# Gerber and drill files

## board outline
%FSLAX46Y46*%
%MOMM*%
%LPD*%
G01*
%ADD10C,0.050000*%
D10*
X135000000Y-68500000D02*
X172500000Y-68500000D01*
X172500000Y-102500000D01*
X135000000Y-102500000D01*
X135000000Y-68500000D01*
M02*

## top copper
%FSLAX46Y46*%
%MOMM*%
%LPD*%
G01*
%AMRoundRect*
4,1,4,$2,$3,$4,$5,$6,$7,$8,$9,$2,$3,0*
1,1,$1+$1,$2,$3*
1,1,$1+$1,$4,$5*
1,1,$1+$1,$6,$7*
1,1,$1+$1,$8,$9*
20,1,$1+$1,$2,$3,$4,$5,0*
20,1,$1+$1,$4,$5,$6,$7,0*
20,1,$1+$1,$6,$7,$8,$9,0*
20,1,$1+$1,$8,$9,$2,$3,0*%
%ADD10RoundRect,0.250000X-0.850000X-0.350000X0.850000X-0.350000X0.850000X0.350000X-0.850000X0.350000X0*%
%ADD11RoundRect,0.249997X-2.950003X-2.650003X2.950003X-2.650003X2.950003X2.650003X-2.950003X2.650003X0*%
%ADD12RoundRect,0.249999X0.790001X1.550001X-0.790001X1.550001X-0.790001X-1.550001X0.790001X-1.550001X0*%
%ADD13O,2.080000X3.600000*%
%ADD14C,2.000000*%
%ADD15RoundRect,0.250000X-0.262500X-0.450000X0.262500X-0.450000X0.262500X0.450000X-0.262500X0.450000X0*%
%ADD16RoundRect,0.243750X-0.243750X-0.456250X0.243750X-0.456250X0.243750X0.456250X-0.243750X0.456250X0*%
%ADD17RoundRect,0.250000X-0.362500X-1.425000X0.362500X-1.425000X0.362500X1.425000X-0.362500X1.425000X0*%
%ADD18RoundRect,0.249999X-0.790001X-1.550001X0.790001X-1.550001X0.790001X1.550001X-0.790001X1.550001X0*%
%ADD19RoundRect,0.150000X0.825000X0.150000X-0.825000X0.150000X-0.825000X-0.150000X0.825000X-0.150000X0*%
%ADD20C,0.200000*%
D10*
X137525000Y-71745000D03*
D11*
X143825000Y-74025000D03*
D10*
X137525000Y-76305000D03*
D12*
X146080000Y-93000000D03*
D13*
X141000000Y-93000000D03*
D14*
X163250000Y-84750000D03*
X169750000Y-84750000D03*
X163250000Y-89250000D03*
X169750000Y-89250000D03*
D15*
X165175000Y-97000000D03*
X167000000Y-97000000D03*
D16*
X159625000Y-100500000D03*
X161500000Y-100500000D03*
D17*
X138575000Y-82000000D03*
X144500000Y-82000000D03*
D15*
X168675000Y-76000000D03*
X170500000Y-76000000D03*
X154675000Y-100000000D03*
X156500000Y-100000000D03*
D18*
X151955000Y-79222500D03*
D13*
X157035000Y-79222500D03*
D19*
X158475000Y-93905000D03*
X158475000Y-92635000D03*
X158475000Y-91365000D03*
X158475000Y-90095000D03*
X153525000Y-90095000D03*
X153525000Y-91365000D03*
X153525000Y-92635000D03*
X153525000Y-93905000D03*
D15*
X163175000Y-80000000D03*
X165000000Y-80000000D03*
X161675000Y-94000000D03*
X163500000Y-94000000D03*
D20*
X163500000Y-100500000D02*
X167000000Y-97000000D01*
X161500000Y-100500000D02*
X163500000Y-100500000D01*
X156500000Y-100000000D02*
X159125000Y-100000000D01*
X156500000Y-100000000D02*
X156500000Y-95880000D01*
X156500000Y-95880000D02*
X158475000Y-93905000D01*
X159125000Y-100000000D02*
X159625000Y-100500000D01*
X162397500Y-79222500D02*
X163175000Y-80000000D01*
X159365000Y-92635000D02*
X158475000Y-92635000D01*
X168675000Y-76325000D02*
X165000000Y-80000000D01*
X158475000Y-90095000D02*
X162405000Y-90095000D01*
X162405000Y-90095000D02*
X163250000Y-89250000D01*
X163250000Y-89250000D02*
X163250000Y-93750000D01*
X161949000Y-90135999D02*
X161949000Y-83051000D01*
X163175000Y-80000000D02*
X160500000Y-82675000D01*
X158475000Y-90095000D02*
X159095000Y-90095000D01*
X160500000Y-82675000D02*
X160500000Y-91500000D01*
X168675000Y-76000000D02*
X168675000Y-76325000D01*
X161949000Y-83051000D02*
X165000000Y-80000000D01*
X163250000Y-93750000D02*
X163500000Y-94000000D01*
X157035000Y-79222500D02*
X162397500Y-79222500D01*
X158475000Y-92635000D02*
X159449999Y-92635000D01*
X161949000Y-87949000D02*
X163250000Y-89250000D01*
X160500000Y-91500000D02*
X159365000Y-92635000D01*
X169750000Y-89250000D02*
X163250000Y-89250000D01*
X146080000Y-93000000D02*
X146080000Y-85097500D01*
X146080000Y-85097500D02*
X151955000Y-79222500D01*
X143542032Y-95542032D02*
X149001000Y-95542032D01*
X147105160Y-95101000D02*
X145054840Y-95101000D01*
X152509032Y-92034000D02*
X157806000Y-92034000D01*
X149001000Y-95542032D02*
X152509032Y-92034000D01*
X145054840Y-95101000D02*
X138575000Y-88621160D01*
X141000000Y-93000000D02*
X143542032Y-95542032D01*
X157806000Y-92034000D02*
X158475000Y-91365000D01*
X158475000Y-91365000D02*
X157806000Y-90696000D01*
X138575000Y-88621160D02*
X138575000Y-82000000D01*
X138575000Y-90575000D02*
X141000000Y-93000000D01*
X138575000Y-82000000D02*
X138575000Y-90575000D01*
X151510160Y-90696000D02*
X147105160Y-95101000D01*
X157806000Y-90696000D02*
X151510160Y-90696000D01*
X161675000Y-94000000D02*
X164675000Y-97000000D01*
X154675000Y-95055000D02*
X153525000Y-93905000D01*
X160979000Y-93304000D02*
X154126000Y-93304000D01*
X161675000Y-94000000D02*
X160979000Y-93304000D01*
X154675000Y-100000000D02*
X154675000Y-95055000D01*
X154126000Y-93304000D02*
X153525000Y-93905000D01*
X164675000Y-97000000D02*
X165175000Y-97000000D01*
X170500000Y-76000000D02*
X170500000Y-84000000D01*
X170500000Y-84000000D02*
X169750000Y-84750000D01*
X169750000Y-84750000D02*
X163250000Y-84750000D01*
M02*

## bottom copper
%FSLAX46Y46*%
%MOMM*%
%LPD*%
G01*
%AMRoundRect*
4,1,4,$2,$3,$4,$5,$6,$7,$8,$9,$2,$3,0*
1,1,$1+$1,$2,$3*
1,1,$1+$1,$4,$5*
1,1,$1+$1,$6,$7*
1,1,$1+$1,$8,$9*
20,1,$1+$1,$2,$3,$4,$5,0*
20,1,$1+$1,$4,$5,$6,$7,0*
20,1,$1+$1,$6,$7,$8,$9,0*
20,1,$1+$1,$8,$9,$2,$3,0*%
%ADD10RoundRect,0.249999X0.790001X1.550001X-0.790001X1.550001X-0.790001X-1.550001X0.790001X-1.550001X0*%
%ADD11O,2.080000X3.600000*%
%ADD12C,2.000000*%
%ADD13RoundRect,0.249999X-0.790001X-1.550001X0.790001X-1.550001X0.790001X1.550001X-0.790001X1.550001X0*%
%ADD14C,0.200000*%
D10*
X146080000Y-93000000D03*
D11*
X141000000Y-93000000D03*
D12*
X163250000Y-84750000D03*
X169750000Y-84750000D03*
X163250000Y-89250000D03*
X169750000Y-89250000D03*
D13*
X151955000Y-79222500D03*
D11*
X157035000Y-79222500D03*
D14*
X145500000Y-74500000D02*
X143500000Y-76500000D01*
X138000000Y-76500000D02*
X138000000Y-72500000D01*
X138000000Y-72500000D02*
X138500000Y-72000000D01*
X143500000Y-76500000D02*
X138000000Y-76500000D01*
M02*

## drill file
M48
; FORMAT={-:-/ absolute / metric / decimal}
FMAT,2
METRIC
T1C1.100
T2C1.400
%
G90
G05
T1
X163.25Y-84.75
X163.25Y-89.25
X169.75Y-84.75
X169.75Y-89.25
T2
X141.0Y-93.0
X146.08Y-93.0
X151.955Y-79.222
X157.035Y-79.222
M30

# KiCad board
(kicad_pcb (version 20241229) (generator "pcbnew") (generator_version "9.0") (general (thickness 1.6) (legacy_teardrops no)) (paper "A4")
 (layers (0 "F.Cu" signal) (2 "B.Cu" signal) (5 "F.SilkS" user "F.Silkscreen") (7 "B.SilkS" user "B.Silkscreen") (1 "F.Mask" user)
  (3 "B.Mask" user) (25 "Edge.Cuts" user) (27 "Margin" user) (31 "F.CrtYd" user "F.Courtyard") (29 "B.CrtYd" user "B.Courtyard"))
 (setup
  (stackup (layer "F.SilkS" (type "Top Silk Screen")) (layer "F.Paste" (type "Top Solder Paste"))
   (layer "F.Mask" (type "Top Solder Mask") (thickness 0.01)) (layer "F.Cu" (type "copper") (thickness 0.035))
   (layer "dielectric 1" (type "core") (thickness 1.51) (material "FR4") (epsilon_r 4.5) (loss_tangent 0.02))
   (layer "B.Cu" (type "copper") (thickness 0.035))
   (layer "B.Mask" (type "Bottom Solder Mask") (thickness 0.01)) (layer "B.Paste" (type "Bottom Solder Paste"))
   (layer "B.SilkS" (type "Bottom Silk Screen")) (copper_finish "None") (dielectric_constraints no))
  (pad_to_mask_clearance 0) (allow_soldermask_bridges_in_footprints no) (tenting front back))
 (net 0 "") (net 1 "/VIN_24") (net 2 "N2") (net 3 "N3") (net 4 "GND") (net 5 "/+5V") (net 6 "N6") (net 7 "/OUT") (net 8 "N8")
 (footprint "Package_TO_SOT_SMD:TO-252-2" (layer "F.Cu") (at 142.565 74.025)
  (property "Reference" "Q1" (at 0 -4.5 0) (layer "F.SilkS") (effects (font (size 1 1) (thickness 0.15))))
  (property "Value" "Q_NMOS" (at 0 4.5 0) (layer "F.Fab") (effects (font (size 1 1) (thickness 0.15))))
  (pad "" smd roundrect (at -0.415 -1.525) (size 3.05 2.75) (layers "F.Paste") (roundrect_rratio 0.090909))
  (pad "" smd roundrect (at -0.415 1.525) (size 3.05 2.75) (layers "F.Paste") (roundrect_rratio 0.090909))
  (pad "" smd roundrect (at 2.935 -1.525) (size 3.05 2.75) (layers "F.Paste") (roundrect_rratio 0.090909))
  (pad "" smd roundrect (at 2.935 1.525) (size 3.05 2.75) (layers "F.Paste") (roundrect_rratio 0.090909))
  (pad "1" smd roundrect (at -5.04 -2.28) (size 2.2 1.2) (layers "F.Cu" "F.Mask" "F.Paste") (roundrect_rratio 0.208333))
  (pad "2" smd roundrect (at 1.26 0) (size 6.4 5.8) (layers "F.Cu" "F.Mask") (roundrect_rratio 0.043103))
  (pad "3" smd roundrect (at -5.04 2.28) (size 2.2 1.2) (layers "F.Cu" "F.Mask" "F.Paste") (roundrect_rratio 0.208333)))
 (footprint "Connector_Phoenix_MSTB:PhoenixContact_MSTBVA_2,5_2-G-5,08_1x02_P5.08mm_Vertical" (layer "F.Cu") (at 146.08 93 180)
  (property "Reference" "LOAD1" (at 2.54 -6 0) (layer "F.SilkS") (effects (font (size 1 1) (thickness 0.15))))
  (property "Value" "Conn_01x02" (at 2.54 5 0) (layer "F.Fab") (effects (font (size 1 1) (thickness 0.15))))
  (pad "1" thru_hole roundrect (at 0 0 180) (size 2.08 3.6) (drill 1.4) (layers "*.Cu" "*.Mask") (remove_unused_layers no)
   (roundrect_rratio 0.120192) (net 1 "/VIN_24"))
  (pad "2" thru_hole oval (at 5.08 0 180) (size 2.08 3.6) (drill 1.4) (layers "*.Cu" "*.Mask") (remove_unused_layers no) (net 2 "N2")))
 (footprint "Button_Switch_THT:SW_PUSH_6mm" (layer "F.Cu") (at 163.25 84.75)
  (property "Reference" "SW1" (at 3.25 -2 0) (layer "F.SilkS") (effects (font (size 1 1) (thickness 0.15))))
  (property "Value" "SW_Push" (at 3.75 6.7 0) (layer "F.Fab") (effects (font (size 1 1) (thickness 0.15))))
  (pad "1" thru_hole circle (at 0 0 90) (size 2 2) (drill 1.1) (layers "*.Cu" "*.Mask") (remove_unused_layers no) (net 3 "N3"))
  (pad "1" thru_hole circle (at 6.5 0 90) (size 2 2) (drill 1.1) (layers "*.Cu" "*.Mask") (remove_unused_layers no) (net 3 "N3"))
  (pad "2" thru_hole circle (at 0 4.5 90) (size 2 2) (drill 1.1) (layers "*.Cu" "*.Mask") (remove_unused_layers no) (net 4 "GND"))
  (pad "2" thru_hole circle (at 6.5 4.5 90) (size 2 2) (drill 1.1) (layers "*.Cu" "*.Mask") (remove_unused_layers no) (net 4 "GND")))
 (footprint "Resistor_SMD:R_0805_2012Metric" (layer "F.Cu") (at 166.0875 97)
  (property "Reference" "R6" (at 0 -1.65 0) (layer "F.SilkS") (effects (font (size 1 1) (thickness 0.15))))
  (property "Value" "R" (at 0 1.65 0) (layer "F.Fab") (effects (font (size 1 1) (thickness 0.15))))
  (pad "1" smd roundrect (at -0.9125 0) (size 1.025 1.4) (layers "F.Cu" "F.Mask" "F.Paste") (roundrect_rratio 0.243902) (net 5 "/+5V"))
  (pad "2" smd roundrect (at 0.9125 0) (size 1.025 1.4) (layers "F.Cu" "F.Mask" "F.Paste") (roundrect_rratio 0.243902) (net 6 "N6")))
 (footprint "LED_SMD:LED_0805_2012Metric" (layer "F.Cu") (at 160.5625 100.5)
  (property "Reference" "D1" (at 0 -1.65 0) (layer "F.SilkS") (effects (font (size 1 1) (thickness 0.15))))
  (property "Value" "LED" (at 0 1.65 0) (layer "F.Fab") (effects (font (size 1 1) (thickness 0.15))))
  (pad "1" smd roundrect (at -0.9375 0) (size 0.975 1.4) (layers "F.Cu" "F.Mask" "F.Paste") (roundrect_rratio 0.25) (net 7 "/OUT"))
  (pad "2" smd roundrect (at 0.9375 0) (size 0.975 1.4) (layers "F.Cu" "F.Mask" "F.Paste") (roundrect_rratio 0.25) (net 6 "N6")))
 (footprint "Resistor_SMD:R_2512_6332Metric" (layer "F.Cu") (at 141.5375 82)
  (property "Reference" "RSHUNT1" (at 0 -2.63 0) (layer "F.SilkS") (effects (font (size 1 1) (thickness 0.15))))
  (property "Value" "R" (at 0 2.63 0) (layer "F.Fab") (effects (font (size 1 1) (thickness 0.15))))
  (pad "1" smd roundrect (at -2.9625 0) (size 1.225 3.35) (layers "F.Cu" "F.Mask" "F.Paste") (roundrect_rratio 0.204082) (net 2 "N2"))
  (pad "2" smd roundrect (at 2.9625 0) (size 1.225 3.35) (layers "F.Cu" "F.Mask" "F.Paste") (roundrect_rratio 0.204082) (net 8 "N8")))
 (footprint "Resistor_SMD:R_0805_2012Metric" (layer "F.Cu") (at 169.5875 76)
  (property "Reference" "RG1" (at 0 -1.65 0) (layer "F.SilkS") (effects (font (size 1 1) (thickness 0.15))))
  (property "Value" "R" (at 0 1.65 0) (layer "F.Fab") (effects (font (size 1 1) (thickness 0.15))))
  (pad "1" smd roundrect (at -0.9125 0) (size 1.025 1.4) (layers "F.Cu" "F.Mask" "F.Paste") (roundrect_rratio 0.243902) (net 4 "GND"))
  (pad "2" smd roundrect (at 0.9125 0) (size 1.025 1.4) (layers "F.Cu" "F.Mask" "F.Paste") (roundrect_rratio 0.243902) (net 3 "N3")))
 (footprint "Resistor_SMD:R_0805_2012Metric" (layer "F.Cu") (at 155.5875 100)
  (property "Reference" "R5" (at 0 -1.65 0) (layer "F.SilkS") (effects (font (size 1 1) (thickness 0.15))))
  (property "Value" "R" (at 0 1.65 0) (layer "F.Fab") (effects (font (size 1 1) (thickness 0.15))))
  (pad "1" smd roundrect (at -0.9125 0) (size 1.025 1.4) (layers "F.Cu" "F.Mask" "F.Paste") (roundrect_rratio 0.243902) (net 5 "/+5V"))
  (pad "2" smd roundrect (at 0.9125 0) (size 1.025 1.4) (layers "F.Cu" "F.Mask" "F.Paste") (roundrect_rratio 0.243902) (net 7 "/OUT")))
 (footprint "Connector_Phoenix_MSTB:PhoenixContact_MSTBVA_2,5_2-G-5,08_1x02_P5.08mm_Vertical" (layer "F.Cu") (at 151.955 79.2225)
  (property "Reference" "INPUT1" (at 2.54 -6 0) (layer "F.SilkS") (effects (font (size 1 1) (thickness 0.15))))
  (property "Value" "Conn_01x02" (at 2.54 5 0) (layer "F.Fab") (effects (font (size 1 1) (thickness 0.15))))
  (pad "1" thru_hole roundrect (at 0 0) (size 2.08 3.6) (drill 1.4) (layers "*.Cu" "*.Mask") (remove_unused_layers no)
   (roundrect_rratio 0.120192) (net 1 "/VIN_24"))
  (pad "2" thru_hole oval (at 5.08 0) (size 2.08 3.6) (drill 1.4) (layers "*.Cu" "*.Mask") (remove_unused_layers no) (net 4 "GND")))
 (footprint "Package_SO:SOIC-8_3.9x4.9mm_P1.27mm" (layer "F.Cu") (at 156 92 180)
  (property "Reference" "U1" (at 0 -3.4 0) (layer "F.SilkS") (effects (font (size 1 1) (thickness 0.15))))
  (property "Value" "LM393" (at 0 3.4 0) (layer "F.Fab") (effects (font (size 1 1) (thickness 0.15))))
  (pad "1" smd roundrect (at -2.475 -1.905 180) (size 1.95 0.6) (layers "F.Cu" "F.Mask" "F.Paste") (roundrect_rratio 0.25) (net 7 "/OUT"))
  (pad "2" smd roundrect (at -2.475 -0.635 180) (size 1.95 0.6) (layers "F.Cu" "F.Mask" "F.Paste") (roundrect_rratio 0.25) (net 4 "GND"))
  (pad "3" smd roundrect (at -2.475 0.635 180) (size 1.95 0.6) (layers "F.Cu" "F.Mask" "F.Paste") (roundrect_rratio 0.25) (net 2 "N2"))
  (pad "4" smd roundrect (at -2.475 1.905 180) (size 1.95 0.6) (layers "F.Cu" "F.Mask" "F.Paste") (roundrect_rratio 0.25) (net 4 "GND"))
  (pad "5" smd roundrect (at 2.475 1.905 180) (size 1.95 0.6) (layers "F.Cu" "F.Mask" "F.Paste") (roundrect_rratio 0.25))
  (pad "6" smd roundrect (at 2.475 0.635 180) (size 1.95 0.6) (layers "F.Cu" "F.Mask" "F.Paste") (roundrect_rratio 0.25))
  (pad "7" smd roundrect (at 2.475 -0.635 180) (size 1.95 0.6) (layers "F.Cu" "F.Mask" "F.Paste") (roundrect_rratio 0.25))
  (pad "8" smd roundrect (at 2.475 -1.905 180) (size 1.95 0.6) (layers "F.Cu" "F.Mask" "F.Paste") (roundrect_rratio 0.25) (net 5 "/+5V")))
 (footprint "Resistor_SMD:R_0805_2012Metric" (layer "F.Cu") (at 164.0875 80)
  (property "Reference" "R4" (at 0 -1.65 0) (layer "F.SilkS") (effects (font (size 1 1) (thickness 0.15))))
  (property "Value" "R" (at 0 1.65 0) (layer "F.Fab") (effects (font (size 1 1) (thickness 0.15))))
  (pad "1" smd roundrect (at -0.9125 0) (size 1.025 1.4) (layers "F.Cu" "F.Mask" "F.Paste") (roundrect_rratio 0.243902) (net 4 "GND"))
  (pad "2" smd roundrect (at 0.9125 0) (size 1.025 1.4) (layers "F.Cu" "F.Mask" "F.Paste") (roundrect_rratio 0.243902) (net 4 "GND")))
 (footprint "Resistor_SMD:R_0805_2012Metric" (layer "F.Cu") (at 162.5875 94)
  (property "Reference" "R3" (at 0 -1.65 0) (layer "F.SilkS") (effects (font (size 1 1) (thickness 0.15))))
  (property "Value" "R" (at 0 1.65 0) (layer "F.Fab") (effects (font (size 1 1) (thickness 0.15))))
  (pad "1" smd roundrect (at -0.9125 0) (size 1.025 1.4) (layers "F.Cu" "F.Mask" "F.Paste") (roundrect_rratio 0.243902) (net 5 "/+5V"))
  (pad "2" smd roundrect (at 0.9125 0) (size 1.025 1.4) (layers "F.Cu" "F.Mask" "F.Paste") (roundrect_rratio 0.243902) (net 4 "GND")))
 (gr_rect (start 135 68.5) (end 172.5 102.5) (stroke (width 0.05) (type default)) (fill no) (layer "Edge.Cuts"))
 (segment (start 145.5 74.5) (end 143.5 76.5) (width 0.2) (layer "B.Cu") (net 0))
 (segment (start 138 76.5) (end 138 72.5) (width 0.2) (layer "B.Cu") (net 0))
 (segment (start 138 72.5) (end 138.5 72) (width 0.2) (layer "B.Cu") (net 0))
 (segment (start 143.5 76.5) (end 138 76.5) (width 0.2) (layer "B.Cu") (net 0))
 (segment (start 163.5 100.5) (end 167 97) (width 0.2) (layer "F.Cu") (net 6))
 (segment (start 161.5 100.5) (end 163.5 100.5) (width 0.2) (layer "F.Cu") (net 6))
 (segment (start 156.5 100) (end 159.125 100) (width 0.2) (layer "F.Cu") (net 7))
 (segment (start 156.5 100) (end 156.5 95.88) (width 0.2) (layer "F.Cu") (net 7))
 (segment (start 156.5 95.88) (end 158.475 93.905) (width 0.2) (layer "F.Cu") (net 7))
 (segment (start 159.125 100) (end 159.625 100.5) (width 0.2) (layer "F.Cu") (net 7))
 (segment (start 162.3975 79.2225) (end 163.175 80) (width 0.2) (layer "F.Cu") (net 4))
 (segment (start 159.365 92.635) (end 158.475 92.635) (width 0.2) (layer "F.Cu") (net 4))
 (segment (start 168.675 76.325) (end 165 80) (width 0.2) (layer "F.Cu") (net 4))
 (segment (start 158.475 90.095) (end 162.405 90.095) (width 0.2) (layer "F.Cu") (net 4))
 (segment (start 162.405 90.095) (end 163.25 89.25) (width 0.2) (layer "F.Cu") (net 4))
 (segment (start 163.25 89.25) (end 163.25 93.75) (width 0.2) (layer "F.Cu") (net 4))
 (segment (start 161.949 90.135999) (end 161.949 83.051) (width 0.2) (layer "F.Cu") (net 4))
 (segment (start 163.175 80) (end 160.5 82.675) (width 0.2) (layer "F.Cu") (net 4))
 (segment (start 158.475 90.095) (end 159.095 90.095) (width 0.2) (layer "F.Cu") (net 4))
 (segment (start 160.5 82.675) (end 160.5 91.5) (width 0.2) (layer "F.Cu") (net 4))
 (segment (start 168.675 76) (end 168.675 76.325) (width 0.2) (layer "F.Cu") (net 4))
 (segment (start 161.949 83.051) (end 165 80) (width 0.2) (layer "F.Cu") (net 4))
 (segment (start 163.25 93.75) (end 163.5 94) (width 0.2) (layer "F.Cu") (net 4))
 (segment (start 157.035 79.2225) (end 162.3975 79.2225) (width 0.2) (layer "F.Cu") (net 4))
 (segment (start 158.475 92.635) (end 159.449999 92.635) (width 0.2) (layer "F.Cu") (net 4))
 (segment (start 161.949 87.949) (end 163.25 89.25) (width 0.2) (layer "F.Cu") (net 4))
 (segment (start 160.5 91.5) (end 159.365 92.635) (width 0.2) (layer "F.Cu") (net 4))
 (segment (start 169.75 89.25) (end 163.25 89.25) (width 0.2) (layer "F.Cu") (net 4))
 (segment (start 146.08 93) (end 146.08 85.0975) (width 0.2) (layer "F.Cu") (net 1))
 (segment (start 146.08 85.0975) (end 151.955 79.2225) (width 0.2) (layer "F.Cu") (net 1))
 (segment (start 143.542032 95.542032) (end 149.001 95.542032) (width 0.2) (layer "F.Cu") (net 2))
 (segment (start 147.10516 95.101) (end 145.05484 95.101) (width 0.2) (layer "F.Cu") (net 2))
 (segment (start 152.509032 92.034) (end 157.806 92.034) (width 0.2) (layer "F.Cu") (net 2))
 (segment (start 149.001 95.542032) (end 152.509032 92.034) (width 0.2) (layer "F.Cu") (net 2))
 (segment (start 145.05484 95.101) (end 138.575 88.62116) (width 0.2) (layer "F.Cu") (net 2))
 (segment (start 141 93) (end 143.542032 95.542032) (width 0.2) (layer "F.Cu") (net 2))
 (segment (start 157.806 92.034) (end 158.475 91.365) (width 0.2) (layer "F.Cu") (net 2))
 (segment (start 158.475 91.365) (end 157.806 90.696) (width 0.2) (layer "F.Cu") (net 2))
 (segment (start 138.575 88.62116) (end 138.575 82) (width 0.2) (layer "F.Cu") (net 2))
 (segment (start 138.575 90.575) (end 141 93) (width 0.2) (layer "F.Cu") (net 2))
 (segment (start 138.575 82) (end 138.575 90.575) (width 0.2) (layer "F.Cu") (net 2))
 (segment (start 151.51016 90.696) (end 147.10516 95.101) (width 0.2) (layer "F.Cu") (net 2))
 (segment (start 157.806 90.696) (end 151.51016 90.696) (width 0.2) (layer "F.Cu") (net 2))
 (segment (start 161.675 94) (end 164.675 97) (width 0.2) (layer "F.Cu") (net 5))
 (segment (start 154.675 95.055) (end 153.525 93.905) (width 0.2) (layer "F.Cu") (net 5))
 (segment (start 160.979 93.304) (end 154.126 93.304) (width 0.2) (layer "F.Cu") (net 5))
 (segment (start 161.675 94) (end 160.979 93.304) (width 0.2) (layer "F.Cu") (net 5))
 (segment (start 154.675 100) (end 154.675 95.055) (width 0.2) (layer "F.Cu") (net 5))
 (segment (start 154.126 93.304) (end 153.525 93.905) (width 0.2) (layer "F.Cu") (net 5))
 (segment (start 164.675 97) (end 165.175 97) (width 0.2) (layer "F.Cu") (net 5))
 (segment (start 170.5 76) (end 170.5 84) (width 0.2) (layer "F.Cu") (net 3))
 (segment (start 170.5 84) (end 169.75 84.75) (width 0.2) (layer "F.Cu") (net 3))
 (segment (start 169.75 84.75) (end 163.25 84.75) (width 0.2) (layer "F.Cu") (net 3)))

